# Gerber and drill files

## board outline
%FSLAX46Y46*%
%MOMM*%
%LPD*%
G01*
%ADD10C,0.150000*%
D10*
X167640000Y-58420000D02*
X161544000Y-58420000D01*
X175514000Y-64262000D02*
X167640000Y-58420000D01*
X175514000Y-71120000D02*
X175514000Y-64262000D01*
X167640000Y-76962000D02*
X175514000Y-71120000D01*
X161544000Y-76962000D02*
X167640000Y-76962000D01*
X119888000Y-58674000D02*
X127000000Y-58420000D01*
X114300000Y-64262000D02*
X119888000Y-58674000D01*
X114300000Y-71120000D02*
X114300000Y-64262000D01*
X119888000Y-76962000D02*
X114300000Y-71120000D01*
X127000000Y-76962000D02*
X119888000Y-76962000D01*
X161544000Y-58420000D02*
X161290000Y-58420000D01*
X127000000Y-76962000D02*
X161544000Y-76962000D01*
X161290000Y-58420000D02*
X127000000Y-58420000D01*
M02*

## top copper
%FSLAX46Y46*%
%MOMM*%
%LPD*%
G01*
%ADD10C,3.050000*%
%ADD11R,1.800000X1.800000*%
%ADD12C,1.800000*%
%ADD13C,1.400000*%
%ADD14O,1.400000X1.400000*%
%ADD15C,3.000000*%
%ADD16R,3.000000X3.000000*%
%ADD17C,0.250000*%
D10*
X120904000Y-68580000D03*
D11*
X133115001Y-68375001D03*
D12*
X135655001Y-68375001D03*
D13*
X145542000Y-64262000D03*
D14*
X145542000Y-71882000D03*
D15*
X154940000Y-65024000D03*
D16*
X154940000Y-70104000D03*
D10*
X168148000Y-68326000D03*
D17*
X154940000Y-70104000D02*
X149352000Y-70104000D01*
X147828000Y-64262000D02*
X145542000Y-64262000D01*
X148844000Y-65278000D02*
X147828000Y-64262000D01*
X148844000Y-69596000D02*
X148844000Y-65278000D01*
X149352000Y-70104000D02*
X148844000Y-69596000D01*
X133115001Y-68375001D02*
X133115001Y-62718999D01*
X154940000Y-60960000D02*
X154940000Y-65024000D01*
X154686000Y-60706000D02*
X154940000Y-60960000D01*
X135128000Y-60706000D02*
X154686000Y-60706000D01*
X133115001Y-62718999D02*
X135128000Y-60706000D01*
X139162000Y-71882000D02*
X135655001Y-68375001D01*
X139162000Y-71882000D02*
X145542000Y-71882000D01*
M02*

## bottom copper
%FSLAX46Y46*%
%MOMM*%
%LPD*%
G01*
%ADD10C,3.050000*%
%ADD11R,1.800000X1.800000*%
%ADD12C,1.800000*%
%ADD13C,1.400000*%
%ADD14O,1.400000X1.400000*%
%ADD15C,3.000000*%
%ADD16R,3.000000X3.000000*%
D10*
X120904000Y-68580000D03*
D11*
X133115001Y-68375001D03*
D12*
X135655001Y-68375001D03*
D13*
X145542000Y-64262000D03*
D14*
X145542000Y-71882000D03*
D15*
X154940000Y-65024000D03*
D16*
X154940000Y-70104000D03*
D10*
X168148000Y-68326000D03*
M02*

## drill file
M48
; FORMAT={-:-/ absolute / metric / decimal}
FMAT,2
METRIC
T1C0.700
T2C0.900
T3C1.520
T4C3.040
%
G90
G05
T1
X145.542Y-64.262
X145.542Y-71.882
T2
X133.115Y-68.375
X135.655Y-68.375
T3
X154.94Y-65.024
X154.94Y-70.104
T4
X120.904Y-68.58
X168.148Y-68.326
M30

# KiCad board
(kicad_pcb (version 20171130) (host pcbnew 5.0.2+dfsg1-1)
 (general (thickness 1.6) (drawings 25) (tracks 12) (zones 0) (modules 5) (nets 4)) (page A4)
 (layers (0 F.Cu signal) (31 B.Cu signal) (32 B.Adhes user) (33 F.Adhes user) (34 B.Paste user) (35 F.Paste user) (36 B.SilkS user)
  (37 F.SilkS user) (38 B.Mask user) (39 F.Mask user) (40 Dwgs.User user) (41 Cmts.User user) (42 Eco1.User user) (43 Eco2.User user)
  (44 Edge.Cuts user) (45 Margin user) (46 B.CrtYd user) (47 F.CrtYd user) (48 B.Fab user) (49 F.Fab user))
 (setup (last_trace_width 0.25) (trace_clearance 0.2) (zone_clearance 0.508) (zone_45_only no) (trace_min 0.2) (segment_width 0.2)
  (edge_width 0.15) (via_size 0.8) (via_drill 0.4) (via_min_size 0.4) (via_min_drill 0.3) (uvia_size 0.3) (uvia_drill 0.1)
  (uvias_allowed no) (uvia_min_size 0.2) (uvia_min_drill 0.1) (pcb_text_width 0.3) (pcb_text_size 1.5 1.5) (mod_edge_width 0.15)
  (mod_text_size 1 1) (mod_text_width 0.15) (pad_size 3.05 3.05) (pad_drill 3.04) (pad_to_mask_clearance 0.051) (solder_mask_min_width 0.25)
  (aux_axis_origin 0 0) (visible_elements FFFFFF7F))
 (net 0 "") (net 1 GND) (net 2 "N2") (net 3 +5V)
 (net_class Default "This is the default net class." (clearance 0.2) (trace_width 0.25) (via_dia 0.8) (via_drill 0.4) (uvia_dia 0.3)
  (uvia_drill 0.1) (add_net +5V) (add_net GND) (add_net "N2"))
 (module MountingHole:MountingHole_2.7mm (layer F.Cu) (at 120.904 68.58)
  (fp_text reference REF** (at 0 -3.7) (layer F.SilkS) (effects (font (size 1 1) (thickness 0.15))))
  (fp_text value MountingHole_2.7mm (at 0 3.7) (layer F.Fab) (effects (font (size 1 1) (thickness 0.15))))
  (pad "" np_thru_hole circle (at 0 0) (size 3.05 3.05) (drill 3.04) (layers *.Cu *.Mask)))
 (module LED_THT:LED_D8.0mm (layer F.Cu) (at 133.115001 68.375001)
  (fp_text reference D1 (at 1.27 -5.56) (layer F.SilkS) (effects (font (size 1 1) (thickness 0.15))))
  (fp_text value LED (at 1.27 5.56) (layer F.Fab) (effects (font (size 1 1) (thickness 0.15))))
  (pad 1 thru_hole rect (at 0 0) (size 1.8 1.8) (drill 0.9) (layers *.Cu *.Mask) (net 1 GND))
  (pad 2 thru_hole circle (at 2.54 0) (size 1.8 1.8) (drill 0.9) (layers *.Cu *.Mask) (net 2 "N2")))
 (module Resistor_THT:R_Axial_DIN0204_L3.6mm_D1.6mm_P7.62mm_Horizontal (layer F.Cu) (at 145.542 64.262 270)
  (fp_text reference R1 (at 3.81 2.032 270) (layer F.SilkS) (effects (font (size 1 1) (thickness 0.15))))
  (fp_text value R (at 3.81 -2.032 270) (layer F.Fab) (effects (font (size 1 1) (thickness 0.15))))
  (pad 1 thru_hole circle (at 0 0 270) (size 1.4 1.4) (drill 0.7) (layers *.Cu *.Mask) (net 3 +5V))
  (pad 2 thru_hole oval (at 7.62 0 270) (size 1.4 1.4) (drill 0.7) (layers *.Cu *.Mask) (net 2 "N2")))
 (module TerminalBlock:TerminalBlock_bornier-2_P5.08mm (layer F.Cu) (at 154.94 70.104 90)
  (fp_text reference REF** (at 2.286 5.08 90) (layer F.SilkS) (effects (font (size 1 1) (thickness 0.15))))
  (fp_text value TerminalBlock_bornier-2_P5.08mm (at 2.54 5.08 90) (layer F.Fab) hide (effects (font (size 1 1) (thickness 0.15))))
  (pad 2 thru_hole circle (at 5.08 0 90) (size 3 3) (drill 1.52) (layers *.Cu *.Mask))
  (pad 1 thru_hole rect (at 0 0 90) (size 3 3) (drill 1.52) (layers *.Cu *.Mask)))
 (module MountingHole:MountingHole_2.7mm (layer F.Cu) (at 168.148 68.326)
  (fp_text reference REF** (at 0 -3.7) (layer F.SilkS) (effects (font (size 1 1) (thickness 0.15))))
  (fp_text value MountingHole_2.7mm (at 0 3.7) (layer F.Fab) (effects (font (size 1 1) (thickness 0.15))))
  (pad "" np_thru_hole circle (at 0 0) (size 3.05 3.05) (drill 3.04) (layers *.Cu *.Mask)))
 (gr_line (start 167.64 58.42) (end 161.544 58.42) (layer Edge.Cuts) (width 0.15))
 (gr_line (start 175.514 64.262) (end 167.64 58.42) (layer Edge.Cuts) (width 0.15))
 (gr_line (start 175.514 71.12) (end 175.514 64.262) (layer Edge.Cuts) (width 0.15))
 (gr_line (start 167.64 76.962) (end 175.514 71.12) (layer Edge.Cuts) (width 0.15))
 (gr_line (start 161.544 76.962) (end 167.64 76.962) (layer Edge.Cuts) (width 0.15))
 (gr_line (start 119.888 58.674) (end 127 58.42) (layer Edge.Cuts) (width 0.15))
 (gr_line (start 114.3 64.262) (end 119.888 58.674) (layer Edge.Cuts) (width 0.15))
 (gr_line (start 114.3 71.12) (end 114.3 64.262) (layer Edge.Cuts) (width 0.15))
 (gr_line (start 119.888 76.962) (end 114.3 71.12) (layer Edge.Cuts) (width 0.15))
 (gr_line (start 127 76.962) (end 119.888 76.962) (layer Edge.Cuts) (width 0.15))
 (gr_line (start 161.544 58.42) (end 161.29 58.42) (layer Edge.Cuts) (width 0.15))
 (gr_line (start 127 76.962) (end 161.544 76.962) (layer Edge.Cuts) (width 0.15))
 (gr_line (start 161.29 58.42) (end 127 58.42) (layer Edge.Cuts) (width 0.15))
 (segment (start 154.94 70.104) (end 149.352 70.104) (width 0.25) (layer F.Cu) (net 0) (status 400000))
 (segment (start 147.828 64.262) (end 145.542 64.262) (width 0.25) (layer F.Cu) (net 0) (status 800000))
 (segment (start 148.844 65.278) (end 147.828 64.262) (width 0.25) (layer F.Cu) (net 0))
 (segment (start 148.844 69.596) (end 148.844 65.278) (width 0.25) (layer F.Cu) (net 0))
 (segment (start 149.352 70.104) (end 148.844 69.596) (width 0.25) (layer F.Cu) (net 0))
 (segment (start 133.115001 68.375001) (end 133.115001 62.718999) (width 0.25) (layer F.Cu) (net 1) (status 400000))
 (segment (start 154.94 60.96) (end 154.94 65.024) (width 0.25) (layer F.Cu) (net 1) (status 800000))
 (segment (start 154.686 60.706) (end 154.94 60.96) (width 0.25) (layer F.Cu) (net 1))
 (segment (start 135.128 60.706) (end 154.686 60.706) (width 0.25) (layer F.Cu) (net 1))
 (segment (start 133.115001 62.718999) (end 135.128 60.706) (width 0.25) (layer F.Cu) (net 1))
 (segment (start 139.162 71.882) (end 135.655001 68.375001) (width 0.25) (layer F.Cu) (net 2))
 (segment (start 139.162 71.882) (end 145.542 71.882) (width 0.25) (layer F.Cu) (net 2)))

